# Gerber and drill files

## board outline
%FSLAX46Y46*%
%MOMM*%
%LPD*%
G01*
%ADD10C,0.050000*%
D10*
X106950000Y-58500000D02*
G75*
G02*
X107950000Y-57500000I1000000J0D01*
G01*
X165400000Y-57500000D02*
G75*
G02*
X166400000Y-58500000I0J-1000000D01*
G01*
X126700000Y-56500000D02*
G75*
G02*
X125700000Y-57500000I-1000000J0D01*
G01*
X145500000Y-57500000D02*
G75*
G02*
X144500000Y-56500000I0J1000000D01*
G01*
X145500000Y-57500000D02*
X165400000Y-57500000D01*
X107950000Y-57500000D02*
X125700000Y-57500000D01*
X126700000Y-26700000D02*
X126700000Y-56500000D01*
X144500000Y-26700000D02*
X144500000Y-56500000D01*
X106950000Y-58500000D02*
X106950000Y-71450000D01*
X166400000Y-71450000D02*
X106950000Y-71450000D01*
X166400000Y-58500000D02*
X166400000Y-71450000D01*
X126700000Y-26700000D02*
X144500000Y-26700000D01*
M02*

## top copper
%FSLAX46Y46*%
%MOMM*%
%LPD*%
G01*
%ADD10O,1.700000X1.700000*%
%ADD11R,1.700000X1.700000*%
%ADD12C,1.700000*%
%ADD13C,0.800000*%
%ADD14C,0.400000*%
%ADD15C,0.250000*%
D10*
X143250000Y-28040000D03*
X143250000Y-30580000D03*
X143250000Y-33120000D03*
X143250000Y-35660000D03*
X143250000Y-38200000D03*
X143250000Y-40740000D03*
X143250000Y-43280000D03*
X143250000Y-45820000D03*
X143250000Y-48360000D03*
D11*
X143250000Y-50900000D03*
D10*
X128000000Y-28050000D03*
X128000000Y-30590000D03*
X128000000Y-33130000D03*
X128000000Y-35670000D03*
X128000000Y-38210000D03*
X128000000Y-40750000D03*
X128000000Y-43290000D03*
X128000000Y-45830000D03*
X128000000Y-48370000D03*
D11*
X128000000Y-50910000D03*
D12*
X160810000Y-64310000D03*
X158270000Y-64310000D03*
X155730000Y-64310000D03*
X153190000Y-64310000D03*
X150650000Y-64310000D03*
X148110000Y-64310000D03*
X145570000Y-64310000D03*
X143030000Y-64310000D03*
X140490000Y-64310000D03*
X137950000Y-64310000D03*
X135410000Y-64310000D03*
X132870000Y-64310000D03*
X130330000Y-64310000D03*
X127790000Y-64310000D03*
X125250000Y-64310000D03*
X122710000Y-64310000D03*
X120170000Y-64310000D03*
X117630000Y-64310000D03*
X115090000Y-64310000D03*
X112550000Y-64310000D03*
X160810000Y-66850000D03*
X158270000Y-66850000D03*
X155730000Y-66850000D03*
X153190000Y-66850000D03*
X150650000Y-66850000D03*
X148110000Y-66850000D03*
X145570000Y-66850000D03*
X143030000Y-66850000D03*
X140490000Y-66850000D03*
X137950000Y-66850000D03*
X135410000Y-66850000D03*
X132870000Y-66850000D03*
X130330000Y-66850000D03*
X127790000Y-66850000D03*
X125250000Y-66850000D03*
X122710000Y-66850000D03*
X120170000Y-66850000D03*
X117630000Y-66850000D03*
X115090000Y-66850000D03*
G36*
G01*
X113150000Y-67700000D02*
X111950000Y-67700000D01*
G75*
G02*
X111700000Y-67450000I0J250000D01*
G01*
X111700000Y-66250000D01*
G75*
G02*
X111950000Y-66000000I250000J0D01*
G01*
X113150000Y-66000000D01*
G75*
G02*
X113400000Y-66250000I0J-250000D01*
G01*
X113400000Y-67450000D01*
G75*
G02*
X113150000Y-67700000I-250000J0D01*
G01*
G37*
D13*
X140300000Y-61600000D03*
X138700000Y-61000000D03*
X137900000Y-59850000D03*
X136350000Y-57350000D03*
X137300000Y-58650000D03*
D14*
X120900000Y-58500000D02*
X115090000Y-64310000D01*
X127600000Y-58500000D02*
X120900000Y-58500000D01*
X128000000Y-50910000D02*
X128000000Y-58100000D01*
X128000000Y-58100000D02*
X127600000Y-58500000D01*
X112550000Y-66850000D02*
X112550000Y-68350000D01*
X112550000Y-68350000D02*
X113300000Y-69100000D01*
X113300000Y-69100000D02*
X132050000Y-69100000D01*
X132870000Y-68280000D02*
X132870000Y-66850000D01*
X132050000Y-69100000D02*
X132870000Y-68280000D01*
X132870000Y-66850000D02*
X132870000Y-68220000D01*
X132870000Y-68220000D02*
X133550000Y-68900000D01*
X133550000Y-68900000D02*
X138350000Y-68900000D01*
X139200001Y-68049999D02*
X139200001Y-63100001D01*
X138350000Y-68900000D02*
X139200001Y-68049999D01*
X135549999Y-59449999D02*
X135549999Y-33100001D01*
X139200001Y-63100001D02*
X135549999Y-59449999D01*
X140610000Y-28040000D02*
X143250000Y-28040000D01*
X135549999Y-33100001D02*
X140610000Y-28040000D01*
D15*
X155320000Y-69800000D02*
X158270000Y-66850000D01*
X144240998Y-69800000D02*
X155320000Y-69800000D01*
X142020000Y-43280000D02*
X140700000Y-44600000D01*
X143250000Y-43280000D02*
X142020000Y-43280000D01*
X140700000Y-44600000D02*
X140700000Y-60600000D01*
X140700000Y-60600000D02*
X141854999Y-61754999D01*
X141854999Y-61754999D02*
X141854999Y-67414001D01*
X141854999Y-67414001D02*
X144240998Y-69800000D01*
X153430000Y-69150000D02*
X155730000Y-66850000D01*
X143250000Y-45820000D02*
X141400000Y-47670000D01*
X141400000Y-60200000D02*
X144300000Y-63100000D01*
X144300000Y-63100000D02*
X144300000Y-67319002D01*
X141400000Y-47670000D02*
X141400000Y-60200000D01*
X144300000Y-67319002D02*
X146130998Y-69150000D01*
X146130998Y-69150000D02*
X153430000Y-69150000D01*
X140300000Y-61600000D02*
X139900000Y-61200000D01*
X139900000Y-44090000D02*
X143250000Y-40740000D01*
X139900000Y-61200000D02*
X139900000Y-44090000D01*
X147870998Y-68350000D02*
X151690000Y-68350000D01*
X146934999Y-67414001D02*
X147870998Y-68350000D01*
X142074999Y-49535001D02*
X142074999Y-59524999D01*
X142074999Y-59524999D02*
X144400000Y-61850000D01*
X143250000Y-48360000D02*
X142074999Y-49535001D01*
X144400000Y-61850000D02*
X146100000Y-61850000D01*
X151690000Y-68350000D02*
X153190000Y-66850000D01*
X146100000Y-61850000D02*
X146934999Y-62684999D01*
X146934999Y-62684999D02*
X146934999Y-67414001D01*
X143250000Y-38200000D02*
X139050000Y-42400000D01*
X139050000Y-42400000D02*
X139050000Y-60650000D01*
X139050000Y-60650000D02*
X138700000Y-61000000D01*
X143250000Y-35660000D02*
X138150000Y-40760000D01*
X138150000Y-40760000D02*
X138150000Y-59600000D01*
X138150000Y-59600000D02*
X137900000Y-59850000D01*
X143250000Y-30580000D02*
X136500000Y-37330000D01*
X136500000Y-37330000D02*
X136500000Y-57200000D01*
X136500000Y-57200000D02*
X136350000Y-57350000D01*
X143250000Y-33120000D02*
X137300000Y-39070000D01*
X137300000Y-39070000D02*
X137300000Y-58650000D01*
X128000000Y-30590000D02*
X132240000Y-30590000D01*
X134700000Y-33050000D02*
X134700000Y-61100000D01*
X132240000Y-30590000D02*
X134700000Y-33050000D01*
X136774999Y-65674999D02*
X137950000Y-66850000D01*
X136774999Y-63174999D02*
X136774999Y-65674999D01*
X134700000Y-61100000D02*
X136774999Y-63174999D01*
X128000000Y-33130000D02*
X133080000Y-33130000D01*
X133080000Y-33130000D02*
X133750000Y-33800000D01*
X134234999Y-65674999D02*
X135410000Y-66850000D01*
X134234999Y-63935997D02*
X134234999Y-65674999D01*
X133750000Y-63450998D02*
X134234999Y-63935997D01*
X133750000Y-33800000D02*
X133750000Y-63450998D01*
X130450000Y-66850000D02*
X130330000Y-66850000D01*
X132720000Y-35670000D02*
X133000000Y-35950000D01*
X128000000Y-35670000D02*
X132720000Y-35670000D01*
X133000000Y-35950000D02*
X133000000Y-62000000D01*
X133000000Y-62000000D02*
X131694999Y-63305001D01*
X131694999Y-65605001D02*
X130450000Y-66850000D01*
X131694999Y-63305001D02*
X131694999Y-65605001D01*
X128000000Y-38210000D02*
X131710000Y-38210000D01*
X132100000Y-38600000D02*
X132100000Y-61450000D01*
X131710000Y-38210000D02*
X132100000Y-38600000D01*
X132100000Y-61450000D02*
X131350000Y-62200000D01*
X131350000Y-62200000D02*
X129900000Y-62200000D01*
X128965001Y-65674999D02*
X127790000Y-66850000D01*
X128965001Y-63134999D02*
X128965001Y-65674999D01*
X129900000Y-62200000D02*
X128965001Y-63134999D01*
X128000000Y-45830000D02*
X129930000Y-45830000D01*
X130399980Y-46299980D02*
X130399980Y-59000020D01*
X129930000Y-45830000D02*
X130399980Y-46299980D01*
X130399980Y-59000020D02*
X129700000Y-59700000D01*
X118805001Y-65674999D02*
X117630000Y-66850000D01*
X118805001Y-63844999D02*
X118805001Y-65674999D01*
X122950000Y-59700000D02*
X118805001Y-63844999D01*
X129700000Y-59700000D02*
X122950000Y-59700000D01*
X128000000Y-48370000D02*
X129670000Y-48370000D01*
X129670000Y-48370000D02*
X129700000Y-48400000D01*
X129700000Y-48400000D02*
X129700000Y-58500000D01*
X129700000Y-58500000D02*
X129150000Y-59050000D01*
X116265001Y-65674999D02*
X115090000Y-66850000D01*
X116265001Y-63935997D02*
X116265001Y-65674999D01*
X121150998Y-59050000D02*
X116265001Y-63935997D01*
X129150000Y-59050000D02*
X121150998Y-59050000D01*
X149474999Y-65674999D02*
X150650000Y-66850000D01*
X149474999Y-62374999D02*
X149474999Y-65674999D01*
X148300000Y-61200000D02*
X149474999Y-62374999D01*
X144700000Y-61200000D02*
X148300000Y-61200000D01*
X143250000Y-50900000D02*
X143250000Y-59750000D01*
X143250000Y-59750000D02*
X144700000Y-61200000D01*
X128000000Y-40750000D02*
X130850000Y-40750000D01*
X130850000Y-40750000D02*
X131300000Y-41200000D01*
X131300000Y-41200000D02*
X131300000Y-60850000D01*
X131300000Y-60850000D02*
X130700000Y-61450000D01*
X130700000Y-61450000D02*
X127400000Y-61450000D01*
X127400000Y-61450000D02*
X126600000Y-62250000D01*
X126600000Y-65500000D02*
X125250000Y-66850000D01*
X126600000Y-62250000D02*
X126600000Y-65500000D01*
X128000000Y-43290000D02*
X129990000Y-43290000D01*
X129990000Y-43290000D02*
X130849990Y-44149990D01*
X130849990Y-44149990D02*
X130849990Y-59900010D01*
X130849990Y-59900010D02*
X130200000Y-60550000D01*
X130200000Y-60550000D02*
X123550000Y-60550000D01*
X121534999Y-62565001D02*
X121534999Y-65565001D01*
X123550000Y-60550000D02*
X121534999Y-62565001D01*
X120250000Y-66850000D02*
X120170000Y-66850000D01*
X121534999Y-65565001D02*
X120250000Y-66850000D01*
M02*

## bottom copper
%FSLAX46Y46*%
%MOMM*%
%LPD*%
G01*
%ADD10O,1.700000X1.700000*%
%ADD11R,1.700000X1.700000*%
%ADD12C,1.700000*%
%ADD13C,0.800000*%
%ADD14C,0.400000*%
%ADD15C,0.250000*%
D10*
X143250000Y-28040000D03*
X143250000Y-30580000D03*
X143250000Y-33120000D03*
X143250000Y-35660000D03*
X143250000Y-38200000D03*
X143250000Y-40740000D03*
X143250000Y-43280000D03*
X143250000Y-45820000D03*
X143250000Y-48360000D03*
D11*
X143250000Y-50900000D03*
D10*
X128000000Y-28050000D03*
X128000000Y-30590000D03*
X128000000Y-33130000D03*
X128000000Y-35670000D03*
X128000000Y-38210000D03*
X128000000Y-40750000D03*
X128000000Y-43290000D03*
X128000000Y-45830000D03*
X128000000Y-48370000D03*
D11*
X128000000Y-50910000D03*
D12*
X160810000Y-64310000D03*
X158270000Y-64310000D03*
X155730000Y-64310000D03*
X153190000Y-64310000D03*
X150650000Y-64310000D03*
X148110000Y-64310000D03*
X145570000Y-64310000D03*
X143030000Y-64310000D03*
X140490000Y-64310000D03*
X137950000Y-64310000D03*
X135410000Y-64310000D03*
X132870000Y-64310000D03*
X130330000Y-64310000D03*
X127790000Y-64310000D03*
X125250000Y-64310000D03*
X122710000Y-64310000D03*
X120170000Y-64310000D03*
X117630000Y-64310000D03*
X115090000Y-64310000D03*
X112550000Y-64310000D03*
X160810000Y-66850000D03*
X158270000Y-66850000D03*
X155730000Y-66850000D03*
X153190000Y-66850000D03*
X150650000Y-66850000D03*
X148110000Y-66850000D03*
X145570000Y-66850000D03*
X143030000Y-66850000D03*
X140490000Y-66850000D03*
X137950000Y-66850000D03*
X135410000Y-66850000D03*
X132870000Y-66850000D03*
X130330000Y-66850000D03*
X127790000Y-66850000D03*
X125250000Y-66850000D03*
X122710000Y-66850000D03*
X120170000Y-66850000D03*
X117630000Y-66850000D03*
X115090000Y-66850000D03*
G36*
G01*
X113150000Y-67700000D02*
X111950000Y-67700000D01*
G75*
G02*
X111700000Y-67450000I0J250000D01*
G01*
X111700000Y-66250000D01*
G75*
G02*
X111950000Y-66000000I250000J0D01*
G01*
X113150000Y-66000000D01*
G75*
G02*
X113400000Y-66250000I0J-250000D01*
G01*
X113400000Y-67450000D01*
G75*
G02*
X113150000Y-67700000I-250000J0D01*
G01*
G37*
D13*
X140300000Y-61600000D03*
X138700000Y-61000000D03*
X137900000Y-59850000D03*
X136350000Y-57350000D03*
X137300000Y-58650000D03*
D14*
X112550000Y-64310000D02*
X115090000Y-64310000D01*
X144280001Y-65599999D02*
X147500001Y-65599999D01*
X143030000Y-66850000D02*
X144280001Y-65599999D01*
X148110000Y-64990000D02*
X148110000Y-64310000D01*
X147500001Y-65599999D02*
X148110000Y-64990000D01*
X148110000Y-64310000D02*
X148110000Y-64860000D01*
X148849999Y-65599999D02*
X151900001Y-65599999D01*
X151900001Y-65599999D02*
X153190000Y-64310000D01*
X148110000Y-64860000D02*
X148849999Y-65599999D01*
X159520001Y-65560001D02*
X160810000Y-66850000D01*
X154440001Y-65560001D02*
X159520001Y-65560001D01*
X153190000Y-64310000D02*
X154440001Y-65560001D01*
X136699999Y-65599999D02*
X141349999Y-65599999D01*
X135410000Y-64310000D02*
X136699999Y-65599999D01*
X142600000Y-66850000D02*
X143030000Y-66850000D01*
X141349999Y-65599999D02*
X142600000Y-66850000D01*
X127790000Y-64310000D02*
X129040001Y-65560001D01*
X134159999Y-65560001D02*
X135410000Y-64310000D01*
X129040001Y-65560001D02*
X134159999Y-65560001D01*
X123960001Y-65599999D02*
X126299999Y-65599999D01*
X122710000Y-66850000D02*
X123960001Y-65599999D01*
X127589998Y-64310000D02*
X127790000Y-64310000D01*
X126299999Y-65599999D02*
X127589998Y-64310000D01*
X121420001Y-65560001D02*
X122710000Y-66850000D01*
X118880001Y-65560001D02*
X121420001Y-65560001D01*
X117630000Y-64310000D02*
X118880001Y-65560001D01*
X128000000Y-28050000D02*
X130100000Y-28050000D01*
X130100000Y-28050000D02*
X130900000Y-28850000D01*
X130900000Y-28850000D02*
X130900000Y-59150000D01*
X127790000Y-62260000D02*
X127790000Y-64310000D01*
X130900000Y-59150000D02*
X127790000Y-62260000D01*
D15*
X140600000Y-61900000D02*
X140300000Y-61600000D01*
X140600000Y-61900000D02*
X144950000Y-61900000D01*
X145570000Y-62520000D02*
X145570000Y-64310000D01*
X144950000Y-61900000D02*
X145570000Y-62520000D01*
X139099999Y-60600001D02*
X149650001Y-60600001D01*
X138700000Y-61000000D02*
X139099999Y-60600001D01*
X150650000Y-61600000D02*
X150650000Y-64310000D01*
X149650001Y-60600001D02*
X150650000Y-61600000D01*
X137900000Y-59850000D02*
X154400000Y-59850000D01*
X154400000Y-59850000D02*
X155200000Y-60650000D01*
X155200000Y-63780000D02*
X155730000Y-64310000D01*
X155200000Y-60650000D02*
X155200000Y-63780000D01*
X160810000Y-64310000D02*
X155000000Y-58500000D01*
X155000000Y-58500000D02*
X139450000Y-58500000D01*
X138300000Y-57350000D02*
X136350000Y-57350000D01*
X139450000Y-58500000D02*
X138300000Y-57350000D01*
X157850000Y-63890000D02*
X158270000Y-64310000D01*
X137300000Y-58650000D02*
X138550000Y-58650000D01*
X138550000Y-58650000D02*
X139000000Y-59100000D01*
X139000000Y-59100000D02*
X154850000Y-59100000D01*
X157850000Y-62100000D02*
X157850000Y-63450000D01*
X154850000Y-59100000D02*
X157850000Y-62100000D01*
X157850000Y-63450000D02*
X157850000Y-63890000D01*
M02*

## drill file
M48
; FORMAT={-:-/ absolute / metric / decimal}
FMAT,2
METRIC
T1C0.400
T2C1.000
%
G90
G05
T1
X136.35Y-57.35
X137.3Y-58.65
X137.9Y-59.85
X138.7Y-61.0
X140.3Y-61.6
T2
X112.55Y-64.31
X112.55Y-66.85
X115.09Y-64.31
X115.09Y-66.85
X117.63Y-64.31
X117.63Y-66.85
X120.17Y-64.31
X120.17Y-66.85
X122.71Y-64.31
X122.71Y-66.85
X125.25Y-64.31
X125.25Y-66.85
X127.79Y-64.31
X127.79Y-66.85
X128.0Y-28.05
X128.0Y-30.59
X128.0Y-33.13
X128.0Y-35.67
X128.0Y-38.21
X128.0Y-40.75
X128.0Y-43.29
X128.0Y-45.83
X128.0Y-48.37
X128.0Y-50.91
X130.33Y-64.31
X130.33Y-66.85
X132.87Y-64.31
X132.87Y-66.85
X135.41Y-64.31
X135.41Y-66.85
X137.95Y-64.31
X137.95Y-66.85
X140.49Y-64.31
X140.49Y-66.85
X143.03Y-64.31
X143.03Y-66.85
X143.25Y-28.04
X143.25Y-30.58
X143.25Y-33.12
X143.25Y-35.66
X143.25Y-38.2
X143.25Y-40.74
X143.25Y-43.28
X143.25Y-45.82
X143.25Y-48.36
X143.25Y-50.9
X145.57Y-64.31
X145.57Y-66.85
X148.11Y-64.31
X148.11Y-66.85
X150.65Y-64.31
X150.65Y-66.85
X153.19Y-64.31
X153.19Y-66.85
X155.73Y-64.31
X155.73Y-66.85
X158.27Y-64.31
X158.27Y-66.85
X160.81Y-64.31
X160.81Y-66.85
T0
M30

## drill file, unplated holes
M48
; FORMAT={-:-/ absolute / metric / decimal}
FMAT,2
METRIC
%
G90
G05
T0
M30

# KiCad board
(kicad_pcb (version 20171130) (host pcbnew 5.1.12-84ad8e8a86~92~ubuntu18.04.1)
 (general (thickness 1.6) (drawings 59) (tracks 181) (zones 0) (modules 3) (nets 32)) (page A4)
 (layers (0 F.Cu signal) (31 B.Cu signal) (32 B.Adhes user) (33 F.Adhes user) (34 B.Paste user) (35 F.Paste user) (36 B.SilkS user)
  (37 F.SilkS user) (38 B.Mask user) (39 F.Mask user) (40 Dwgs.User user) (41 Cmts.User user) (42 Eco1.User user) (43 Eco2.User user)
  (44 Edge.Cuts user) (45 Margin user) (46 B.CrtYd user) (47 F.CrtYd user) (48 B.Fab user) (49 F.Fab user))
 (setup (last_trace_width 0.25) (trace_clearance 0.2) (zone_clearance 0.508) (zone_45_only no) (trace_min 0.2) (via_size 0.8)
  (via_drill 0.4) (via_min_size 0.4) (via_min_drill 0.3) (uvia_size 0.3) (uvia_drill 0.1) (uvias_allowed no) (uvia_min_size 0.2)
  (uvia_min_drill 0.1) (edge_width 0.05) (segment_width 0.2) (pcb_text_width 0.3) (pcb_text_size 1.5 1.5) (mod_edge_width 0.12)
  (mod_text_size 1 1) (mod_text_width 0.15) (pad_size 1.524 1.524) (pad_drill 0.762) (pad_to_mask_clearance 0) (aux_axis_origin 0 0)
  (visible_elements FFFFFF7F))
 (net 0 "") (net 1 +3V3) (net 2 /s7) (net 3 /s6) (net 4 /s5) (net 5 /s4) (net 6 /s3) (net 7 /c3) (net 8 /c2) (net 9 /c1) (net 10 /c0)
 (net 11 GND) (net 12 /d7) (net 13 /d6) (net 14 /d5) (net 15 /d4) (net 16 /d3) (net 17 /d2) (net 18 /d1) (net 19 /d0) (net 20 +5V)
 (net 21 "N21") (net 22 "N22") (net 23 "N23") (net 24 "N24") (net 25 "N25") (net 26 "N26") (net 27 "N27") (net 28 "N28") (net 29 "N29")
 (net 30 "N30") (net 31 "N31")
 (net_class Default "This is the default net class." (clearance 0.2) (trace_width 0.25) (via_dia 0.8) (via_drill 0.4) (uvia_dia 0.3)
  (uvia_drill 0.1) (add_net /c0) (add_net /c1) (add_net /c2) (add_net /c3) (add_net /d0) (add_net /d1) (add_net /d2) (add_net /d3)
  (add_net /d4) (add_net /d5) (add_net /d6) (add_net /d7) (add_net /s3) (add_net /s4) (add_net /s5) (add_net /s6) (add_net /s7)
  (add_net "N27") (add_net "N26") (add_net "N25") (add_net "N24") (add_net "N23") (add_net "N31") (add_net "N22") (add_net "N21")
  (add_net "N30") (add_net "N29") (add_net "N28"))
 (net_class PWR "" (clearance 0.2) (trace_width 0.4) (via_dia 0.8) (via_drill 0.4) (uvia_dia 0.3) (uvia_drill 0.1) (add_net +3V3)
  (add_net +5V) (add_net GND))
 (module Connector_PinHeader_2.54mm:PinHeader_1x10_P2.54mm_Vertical (layer F.Cu) (at 143.25 50.9 180)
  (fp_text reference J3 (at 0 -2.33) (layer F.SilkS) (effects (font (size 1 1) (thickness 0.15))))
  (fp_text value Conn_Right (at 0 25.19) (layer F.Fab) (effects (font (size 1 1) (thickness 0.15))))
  (pad 10 thru_hole oval (at 0 22.86 180) (size 1.7 1.7) (drill 1) (layers *.Cu *.Mask) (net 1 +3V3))
  (pad 9 thru_hole oval (at 0 20.32 180) (size 1.7 1.7) (drill 1) (layers *.Cu *.Mask) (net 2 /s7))
  (pad 8 thru_hole oval (at 0 17.78 180) (size 1.7 1.7) (drill 1) (layers *.Cu *.Mask) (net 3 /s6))
  (pad 7 thru_hole oval (at 0 15.24 180) (size 1.7 1.7) (drill 1) (layers *.Cu *.Mask) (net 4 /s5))
  (pad 6 thru_hole oval (at 0 12.7 180) (size 1.7 1.7) (drill 1) (layers *.Cu *.Mask) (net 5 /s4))
  (pad 5 thru_hole oval (at 0 10.16 180) (size 1.7 1.7) (drill 1) (layers *.Cu *.Mask) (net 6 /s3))
  (pad 4 thru_hole oval (at 0 7.62 180) (size 1.7 1.7) (drill 1) (layers *.Cu *.Mask) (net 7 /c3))
  (pad 3 thru_hole oval (at 0 5.08 180) (size 1.7 1.7) (drill 1) (layers *.Cu *.Mask) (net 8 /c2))
  (pad 2 thru_hole oval (at 0 2.54 180) (size 1.7 1.7) (drill 1) (layers *.Cu *.Mask) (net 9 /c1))
  (pad 1 thru_hole rect (at 0 0 180) (size 1.7 1.7) (drill 1) (layers *.Cu *.Mask) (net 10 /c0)))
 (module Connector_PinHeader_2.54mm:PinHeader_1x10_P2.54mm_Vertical (layer F.Cu) (at 128 50.91 180)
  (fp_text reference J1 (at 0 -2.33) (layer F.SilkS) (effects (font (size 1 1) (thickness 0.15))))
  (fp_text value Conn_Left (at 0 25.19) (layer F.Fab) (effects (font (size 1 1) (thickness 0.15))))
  (pad 10 thru_hole oval (at 0 22.86 180) (size 1.7 1.7) (drill 1) (layers *.Cu *.Mask) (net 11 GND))
  (pad 9 thru_hole oval (at 0 20.32 180) (size 1.7 1.7) (drill 1) (layers *.Cu *.Mask) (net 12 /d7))
  (pad 8 thru_hole oval (at 0 17.78 180) (size 1.7 1.7) (drill 1) (layers *.Cu *.Mask) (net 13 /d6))
  (pad 7 thru_hole oval (at 0 15.24 180) (size 1.7 1.7) (drill 1) (layers *.Cu *.Mask) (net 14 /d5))
  (pad 6 thru_hole oval (at 0 12.7 180) (size 1.7 1.7) (drill 1) (layers *.Cu *.Mask) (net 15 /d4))
  (pad 5 thru_hole oval (at 0 10.16 180) (size 1.7 1.7) (drill 1) (layers *.Cu *.Mask) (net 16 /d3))
  (pad 4 thru_hole oval (at 0 7.62 180) (size 1.7 1.7) (drill 1) (layers *.Cu *.Mask) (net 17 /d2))
  (pad 3 thru_hole oval (at 0 5.08 180) (size 1.7 1.7) (drill 1) (layers *.Cu *.Mask) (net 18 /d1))
  (pad 2 thru_hole oval (at 0 2.54 180) (size 1.7 1.7) (drill 1) (layers *.Cu *.Mask) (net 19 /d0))
  (pad 1 thru_hole rect (at 0 0 180) (size 1.7 1.7) (drill 1) (layers *.Cu *.Mask) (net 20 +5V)))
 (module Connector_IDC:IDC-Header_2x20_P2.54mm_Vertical (layer F.Cu) (at 112.55 66.85 90)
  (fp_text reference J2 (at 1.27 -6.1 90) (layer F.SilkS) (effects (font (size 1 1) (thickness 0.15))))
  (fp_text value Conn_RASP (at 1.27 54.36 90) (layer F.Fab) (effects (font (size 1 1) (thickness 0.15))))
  (pad 40 thru_hole circle (at 2.54 48.26 90) (size 1.7 1.7) (drill 1) (layers *.Cu *.Mask) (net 2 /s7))
  (pad 38 thru_hole circle (at 2.54 45.72 90) (size 1.7 1.7) (drill 1) (layers *.Cu *.Mask) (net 3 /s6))
  (pad 36 thru_hole circle (at 2.54 43.18 90) (size 1.7 1.7) (drill 1) (layers *.Cu *.Mask) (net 4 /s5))
  (pad 34 thru_hole circle (at 2.54 40.64 90) (size 1.7 1.7) (drill 1) (layers *.Cu *.Mask) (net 11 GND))
  (pad 32 thru_hole circle (at 2.54 38.1 90) (size 1.7 1.7) (drill 1) (layers *.Cu *.Mask) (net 5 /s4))
  (pad 30 thru_hole circle (at 2.54 35.56 90) (size 1.7 1.7) (drill 1) (layers *.Cu *.Mask) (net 11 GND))
  (pad 28 thru_hole circle (at 2.54 33.02 90) (size 1.7 1.7) (drill 1) (layers *.Cu *.Mask) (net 6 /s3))
  (pad 26 thru_hole circle (at 2.54 30.48 90) (size 1.7 1.7) (drill 1) (layers *.Cu *.Mask) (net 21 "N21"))
  (pad 24 thru_hole circle (at 2.54 27.94 90) (size 1.7 1.7) (drill 1) (layers *.Cu *.Mask) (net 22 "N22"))
  (pad 22 thru_hole circle (at 2.54 25.4 90) (size 1.7 1.7) (drill 1) (layers *.Cu *.Mask) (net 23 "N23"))
  (pad 20 thru_hole circle (at 2.54 22.86 90) (size 1.7 1.7) (drill 1) (layers *.Cu *.Mask) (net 11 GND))
  (pad 18 thru_hole circle (at 2.54 20.32 90) (size 1.7 1.7) (drill 1) (layers *.Cu *.Mask) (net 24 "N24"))
  (pad 16 thru_hole circle (at 2.54 17.78 90) (size 1.7 1.7) (drill 1) (layers *.Cu *.Mask) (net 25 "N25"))
  (pad 14 thru_hole circle (at 2.54 15.24 90) (size 1.7 1.7) (drill 1) (layers *.Cu *.Mask) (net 11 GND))
  (pad 12 thru_hole circle (at 2.54 12.7 90) (size 1.7 1.7) (drill 1) (layers *.Cu *.Mask) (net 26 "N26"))
  (pad 10 thru_hole circle (at 2.54 10.16 90) (size 1.7 1.7) (drill 1) (layers *.Cu *.Mask) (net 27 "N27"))
  (pad 8 thru_hole circle (at 2.54 7.62 90) (size 1.7 1.7) (drill 1) (layers *.Cu *.Mask) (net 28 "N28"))
  (pad 6 thru_hole circle (at 2.54 5.08 90) (size 1.7 1.7) (drill 1) (layers *.Cu *.Mask) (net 11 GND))
  (pad 4 thru_hole circle (at 2.54 2.54 90) (size 1.7 1.7) (drill 1) (layers *.Cu *.Mask) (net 20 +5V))
  (pad 2 thru_hole circle (at 2.54 0 90) (size 1.7 1.7) (drill 1) (layers *.Cu *.Mask) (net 20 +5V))
  (pad 39 thru_hole circle (at 0 48.26 90) (size 1.7 1.7) (drill 1) (layers *.Cu *.Mask) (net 11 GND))
  (pad 37 thru_hole circle (at 0 45.72 90) (size 1.7 1.7) (drill 1) (layers *.Cu *.Mask) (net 7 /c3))
  (pad 35 thru_hole circle (at 0 43.18 90) (size 1.7 1.7) (drill 1) (layers *.Cu *.Mask) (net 8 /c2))
  (pad 33 thru_hole circle (at 0 40.64 90) (size 1.7 1.7) (drill 1) (layers *.Cu *.Mask) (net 9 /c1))
  (pad 31 thru_hole circle (at 0 38.1 90) (size 1.7 1.7) (drill 1) (layers *.Cu *.Mask) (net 10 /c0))
  (pad 29 thru_hole circle (at 0 35.56 90) (size 1.7 1.7) (drill 1) (layers *.Cu *.Mask) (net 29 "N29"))
  (pad 27 thru_hole circle (at 0 33.02 90) (size 1.7 1.7) (drill 1) (layers *.Cu *.Mask) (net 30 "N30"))
  (pad 25 thru_hole circle (at 0 30.48 90) (size 1.7 1.7) (drill 1) (layers *.Cu *.Mask) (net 11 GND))
  (pad 23 thru_hole circle (at 0 27.94 90) (size 1.7 1.7) (drill 1) (layers *.Cu *.Mask) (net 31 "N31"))
  (pad 21 thru_hole circle (at 0 25.4 90) (size 1.7 1.7) (drill 1) (layers *.Cu *.Mask) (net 12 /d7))
  (pad 19 thru_hole circle (at 0 22.86 90) (size 1.7 1.7) (drill 1) (layers *.Cu *.Mask) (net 13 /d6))
  (pad 17 thru_hole circle (at 0 20.32 90) (size 1.7 1.7) (drill 1) (layers *.Cu *.Mask) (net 1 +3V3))
  (pad 15 thru_hole circle (at 0 17.78 90) (size 1.7 1.7) (drill 1) (layers *.Cu *.Mask) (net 14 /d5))
  (pad 13 thru_hole circle (at 0 15.24 90) (size 1.7 1.7) (drill 1) (layers *.Cu *.Mask) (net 15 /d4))
  (pad 11 thru_hole circle (at 0 12.7 90) (size 1.7 1.7) (drill 1) (layers *.Cu *.Mask) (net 16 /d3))
  (pad 9 thru_hole circle (at 0 10.16 90) (size 1.7 1.7) (drill 1) (layers *.Cu *.Mask) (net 11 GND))
  (pad 7 thru_hole circle (at 0 7.62 90) (size 1.7 1.7) (drill 1) (layers *.Cu *.Mask) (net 17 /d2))
  (pad 5 thru_hole circle (at 0 5.08 90) (size 1.7 1.7) (drill 1) (layers *.Cu *.Mask) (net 18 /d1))
  (pad 3 thru_hole circle (at 0 2.54 90) (size 1.7 1.7) (drill 1) (layers *.Cu *.Mask) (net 19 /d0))
  (pad 1 thru_hole roundrect (at 0 0 90) (size 1.7 1.7) (drill 1) (layers *.Cu *.Mask) (roundrect_rratio 0.1470588235294118) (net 1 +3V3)))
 (gr_arc (start 107.95 58.5) (end 107.95 57.5) (angle -90) (layer Edge.Cuts) (width 0.05))
 (gr_arc (start 165.4 58.5) (end 166.4 58.5) (angle -90) (layer Edge.Cuts) (width 0.05))
 (gr_arc (start 125.7 56.5) (end 125.7 57.5) (angle -90) (layer Edge.Cuts) (width 0.05))
 (gr_arc (start 145.5 56.5) (end 144.5 56.5) (angle -90) (layer Edge.Cuts) (width 0.05))
 (gr_line (start 145.5 57.5) (end 165.4 57.5) (layer Edge.Cuts) (width 0.05))
 (gr_line (start 107.95 57.5) (end 125.7 57.5) (layer Edge.Cuts) (width 0.05))
 (gr_line (start 126.7 26.7) (end 126.7 56.5) (layer Edge.Cuts) (width 0.05))
 (gr_line (start 144.5 26.7) (end 144.5 56.5) (layer Edge.Cuts) (width 0.05))
 (gr_line (start 106.95 58.5) (end 106.95 71.45) (layer Edge.Cuts) (width 0.05))
 (gr_line (start 166.4 71.45) (end 106.95 71.45) (layer Edge.Cuts) (width 0.05))
 (gr_line (start 166.4 58.5) (end 166.4 71.45) (layer Edge.Cuts) (width 0.05))
 (gr_line (start 126.7 26.7) (end 144.5 26.7) (layer Edge.Cuts) (width 0.05))
 (segment (start 112.55 64.31) (end 115.09 64.31) (width 0.4) (layer B.Cu) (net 20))
 (segment (start 120.9 58.5) (end 115.09 64.31) (width 0.4) (layer F.Cu) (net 20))
 (segment (start 127.6 58.5) (end 120.9 58.5) (width 0.4) (layer F.Cu) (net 20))
 (segment (start 128 50.91) (end 128 58.1) (width 0.4) (layer F.Cu) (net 20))
 (segment (start 128 58.1) (end 127.6 58.5) (width 0.4) (layer F.Cu) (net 20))
 (segment (start 144.280001 65.599999) (end 147.500001 65.599999) (width 0.4) (layer B.Cu) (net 11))
 (segment (start 143.03 66.85) (end 144.280001 65.599999) (width 0.4) (layer B.Cu) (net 11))
 (segment (start 148.11 64.99) (end 148.11 64.31) (width 0.4) (layer B.Cu) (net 11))
 (segment (start 147.500001 65.599999) (end 148.11 64.99) (width 0.4) (layer B.Cu) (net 11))
 (segment (start 148.11 64.31) (end 148.11 64.86) (width 0.4) (layer B.Cu) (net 11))
 (segment (start 148.849999 65.599999) (end 151.900001 65.599999) (width 0.4) (layer B.Cu) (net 11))
 (segment (start 151.900001 65.599999) (end 153.19 64.31) (width 0.4) (layer B.Cu) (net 11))
 (segment (start 148.11 64.86) (end 148.849999 65.599999) (width 0.4) (layer B.Cu) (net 11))
 (segment (start 159.520001 65.560001) (end 160.81 66.85) (width 0.4) (layer B.Cu) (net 11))
 (segment (start 154.440001 65.560001) (end 159.520001 65.560001) (width 0.4) (layer B.Cu) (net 11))
 (segment (start 153.19 64.31) (end 154.440001 65.560001) (width 0.4) (layer B.Cu) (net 11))
 (segment (start 136.699999 65.599999) (end 141.349999 65.599999) (width 0.4) (layer B.Cu) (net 11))
 (segment (start 135.41 64.31) (end 136.699999 65.599999) (width 0.4) (layer B.Cu) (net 11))
 (segment (start 142.6 66.85) (end 143.03 66.85) (width 0.4) (layer B.Cu) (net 11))
 (segment (start 141.349999 65.599999) (end 142.6 66.85) (width 0.4) (layer B.Cu) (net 11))
 (segment (start 127.79 64.31) (end 129.040001 65.560001) (width 0.4) (layer B.Cu) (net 11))
 (segment (start 134.159999 65.560001) (end 135.41 64.31) (width 0.4) (layer B.Cu) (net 11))
 (segment (start 129.040001 65.560001) (end 134.159999 65.560001) (width 0.4) (layer B.Cu) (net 11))
 (segment (start 123.960001 65.599999) (end 126.299999 65.599999) (width 0.4) (layer B.Cu) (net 11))
 (segment (start 122.71 66.85) (end 123.960001 65.599999) (width 0.4) (layer B.Cu) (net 11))
 (segment (start 127.589998 64.31) (end 127.79 64.31) (width 0.4) (layer B.Cu) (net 11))
 (segment (start 126.299999 65.599999) (end 127.589998 64.31) (width 0.4) (layer B.Cu) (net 11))
 (segment (start 121.420001 65.560001) (end 122.71 66.85) (width 0.4) (layer B.Cu) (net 11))
 (segment (start 118.880001 65.560001) (end 121.420001 65.560001) (width 0.4) (layer B.Cu) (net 11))
 (segment (start 117.63 64.31) (end 118.880001 65.560001) (width 0.4) (layer B.Cu) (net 11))
 (segment (start 128 28.05) (end 130.1 28.05) (width 0.4) (layer B.Cu) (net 11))
 (segment (start 130.1 28.05) (end 130.9 28.85) (width 0.4) (layer B.Cu) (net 11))
 (segment (start 130.9 28.85) (end 130.9 59.15) (width 0.4) (layer B.Cu) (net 11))
 (segment (start 127.79 62.26) (end 127.79 64.31) (width 0.4) (layer B.Cu) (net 11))
 (segment (start 130.9 59.15) (end 127.79 62.26) (width 0.4) (layer B.Cu) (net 11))
 (segment (start 112.55 66.85) (end 112.55 68.35) (width 0.4) (layer F.Cu) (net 1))
 (segment (start 112.55 68.35) (end 113.3 69.1) (width 0.4) (layer F.Cu) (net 1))
 (segment (start 113.3 69.1) (end 132.05 69.1) (width 0.4) (layer F.Cu) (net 1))
 (segment (start 132.87 68.28) (end 132.87 66.85) (width 0.4) (layer F.Cu) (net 1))
 (segment (start 132.05 69.1) (end 132.87 68.28) (width 0.4) (layer F.Cu) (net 1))
 (segment (start 132.87 66.85) (end 132.87 68.22) (width 0.4) (layer F.Cu) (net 1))
 (segment (start 132.87 68.22) (end 133.55 68.9) (width 0.4) (layer F.Cu) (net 1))
 (segment (start 133.55 68.9) (end 138.35 68.9) (width 0.4) (layer F.Cu) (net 1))
 (segment (start 139.200001 68.049999) (end 139.200001 63.100001) (width 0.4) (layer F.Cu) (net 1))
 (segment (start 138.35 68.9) (end 139.200001 68.049999) (width 0.4) (layer F.Cu) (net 1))
 (segment (start 135.549999 59.449999) (end 135.549999 33.100001) (width 0.4) (layer F.Cu) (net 1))
 (segment (start 139.200001 63.100001) (end 135.549999 59.449999) (width 0.4) (layer F.Cu) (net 1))
 (segment (start 140.61 28.04) (end 143.25 28.04) (width 0.4) (layer F.Cu) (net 1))
 (segment (start 135.549999 33.100001) (end 140.61 28.04) (width 0.4) (layer F.Cu) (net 1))
 (segment (start 155.32 69.8) (end 158.27 66.85) (width 0.25) (layer F.Cu) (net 7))
 (segment (start 144.240998 69.8) (end 155.32 69.8) (width 0.25) (layer F.Cu) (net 7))
 (segment (start 142.02 43.28) (end 140.7 44.6) (width 0.25) (layer F.Cu) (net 7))
 (segment (start 143.25 43.28) (end 142.02 43.28) (width 0.25) (layer F.Cu) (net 7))
 (segment (start 140.7 44.6) (end 140.7 60.6) (width 0.25) (layer F.Cu) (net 7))
 (segment (start 140.7 60.6) (end 141.854999 61.754999) (width 0.25) (layer F.Cu) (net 7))
 (segment (start 141.854999 61.754999) (end 141.854999 67.414001) (width 0.25) (layer F.Cu) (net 7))
 (segment (start 141.854999 67.414001) (end 144.240998 69.8) (width 0.25) (layer F.Cu) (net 7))
 (segment (start 153.43 69.15) (end 155.73 66.85) (width 0.25) (layer F.Cu) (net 8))
 (segment (start 143.25 45.82) (end 141.4 47.67) (width 0.25) (layer F.Cu) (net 8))
 (segment (start 141.4 60.2) (end 144.3 63.1) (width 0.25) (layer F.Cu) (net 8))
 (segment (start 144.3 63.1) (end 144.3 67.319002) (width 0.25) (layer F.Cu) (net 8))
 (segment (start 141.4 47.67) (end 141.4 60.2) (width 0.25) (layer F.Cu) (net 8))
 (segment (start 144.3 67.319002) (end 146.130998 69.15) (width 0.25) (layer F.Cu) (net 8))
 (segment (start 146.130998 69.15) (end 153.43 69.15) (width 0.25) (layer F.Cu) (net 8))
 (via (at 140.3 61.6) (size 0.8) (drill 0.4) (layers F.Cu B.Cu) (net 6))
 (segment (start 140.6 61.9) (end 140.3 61.6) (width 0.25) (layer B.Cu) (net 6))
 (segment (start 140.3 61.6) (end 139.9 61.2) (width 0.25) (layer F.Cu) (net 6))
 (segment (start 139.9 44.09) (end 143.25 40.74) (width 0.25) (layer F.Cu) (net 6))
 (segment (start 139.9 61.2) (end 139.9 44.09) (width 0.25) (layer F.Cu) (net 6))
 (segment (start 140.6 61.9) (end 144.95 61.9) (width 0.25) (layer B.Cu) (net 6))
 (segment (start 145.57 62.52) (end 145.57 64.31) (width 0.25) (layer B.Cu) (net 6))
 (segment (start 144.95 61.9) (end 145.57 62.52) (width 0.25) (layer B.Cu) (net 6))
 (segment (start 147.870998 68.35) (end 151.69 68.35) (width 0.25) (layer F.Cu) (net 9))
 (segment (start 146.934999 67.414001) (end 147.870998 68.35) (width 0.25) (layer F.Cu) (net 9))
 (segment (start 142.074999 49.535001) (end 142.074999 59.524999) (width 0.25) (layer F.Cu) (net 9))
 (segment (start 142.074999 59.524999) (end 144.4 61.85) (width 0.25) (layer F.Cu) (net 9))
 (segment (start 143.25 48.36) (end 142.074999 49.535001) (width 0.25) (layer F.Cu) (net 9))
 (segment (start 144.4 61.85) (end 146.1 61.85) (width 0.25) (layer F.Cu) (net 9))
 (segment (start 151.69 68.35) (end 153.19 66.85) (width 0.25) (layer F.Cu) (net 9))
 (segment (start 146.1 61.85) (end 146.934999 62.684999) (width 0.25) (layer F.Cu) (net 9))
 (segment (start 146.934999 62.684999) (end 146.934999 67.414001) (width 0.25) (layer F.Cu) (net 9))
 (segment (start 143.25 38.2) (end 139.05 42.4) (width 0.25) (layer F.Cu) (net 5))
 (via (at 138.7 61) (size 0.8) (drill 0.4) (layers F.Cu B.Cu) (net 5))
 (segment (start 139.05 42.4) (end 139.05 60.65) (width 0.25) (layer F.Cu) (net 5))
 (segment (start 139.05 60.65) (end 138.7 61) (width 0.25) (layer F.Cu) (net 5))
 (segment (start 139.099999 60.600001) (end 149.650001 60.600001) (width 0.25) (layer B.Cu) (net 5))
 (segment (start 138.7 61) (end 139.099999 60.600001) (width 0.25) (layer B.Cu) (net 5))
 (segment (start 150.65 61.6) (end 150.65 64.31) (width 0.25) (layer B.Cu) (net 5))
 (segment (start 149.650001 60.600001) (end 150.65 61.6) (width 0.25) (layer B.Cu) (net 5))
 (segment (start 143.25 35.66) (end 138.15 40.76) (width 0.25) (layer F.Cu) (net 4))
 (segment (start 138.15 40.76) (end 138.15 59.6) (width 0.25) (layer F.Cu) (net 4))
 (via (at 137.9 59.85) (size 0.8) (drill 0.4) (layers F.Cu B.Cu) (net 4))
 (segment (start 138.15 59.6) (end 137.9 59.85) (width 0.25) (layer F.Cu) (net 4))
 (segment (start 137.9 59.85) (end 154.4 59.85) (width 0.25) (layer B.Cu) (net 4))
 (segment (start 154.4 59.85) (end 155.2 60.65) (width 0.25) (layer B.Cu) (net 4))
 (segment (start 155.2 63.78) (end 155.73 64.31) (width 0.25) (layer B.Cu) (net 4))
 (segment (start 155.2 60.65) (end 155.2 63.78) (width 0.25) (layer B.Cu) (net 4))
 (segment (start 143.25 30.58) (end 136.5 37.33) (width 0.25) (layer F.Cu) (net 2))
 (via (at 136.35 57.35) (size 0.8) (drill 0.4) (layers F.Cu B.Cu) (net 2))
 (segment (start 136.5 37.33) (end 136.5 57.2) (width 0.25) (layer F.Cu) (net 2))
 (segment (start 136.5 57.2) (end 136.35 57.35) (width 0.25) (layer F.Cu) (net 2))
 (segment (start 160.81 64.31) (end 155 58.5) (width 0.25) (layer B.Cu) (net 2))
 (segment (start 155 58.5) (end 139.45 58.5) (width 0.25) (layer B.Cu) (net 2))
 (segment (start 138.3 57.35) (end 136.35 57.35) (width 0.25) (layer B.Cu) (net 2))
 (segment (start 139.45 58.5) (end 138.3 57.35) (width 0.25) (layer B.Cu) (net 2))
 (segment (start 143.25 33.12) (end 137.3 39.07) (width 0.25) (layer F.Cu) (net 3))
 (via (at 137.3 58.65) (size 0.8) (drill 0.4) (layers F.Cu B.Cu) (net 3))
 (segment (start 137.3 39.07) (end 137.3 58.65) (width 0.25) (layer F.Cu) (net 3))
 (segment (start 157.85 63.89) (end 158.27 64.31) (width 0.25) (layer B.Cu) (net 3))
 (segment (start 137.3 58.65) (end 138.55 58.65) (width 0.25) (layer B.Cu) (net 3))
 (segment (start 138.55 58.65) (end 139 59.1) (width 0.25) (layer B.Cu) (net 3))
 (segment (start 139 59.1) (end 154.85 59.1) (width 0.25) (layer B.Cu) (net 3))
 (segment (start 157.85 62.1) (end 157.85 63.45) (width 0.25) (layer B.Cu) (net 3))
 (segment (start 154.85 59.1) (end 157.85 62.1) (width 0.25) (layer B.Cu) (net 3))
 (segment (start 157.85 63.45) (end 157.85 63.89) (width 0.25) (layer B.Cu) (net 3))
 (segment (start 128 30.59) (end 132.24 30.59) (width 0.25) (layer F.Cu) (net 12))
 (segment (start 134.7 33.05) (end 134.7 61.1) (width 0.25) (layer F.Cu) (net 12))
 (segment (start 132.24 30.59) (end 134.7 33.05) (width 0.25) (layer F.Cu) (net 12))
 (segment (start 136.774999 65.674999) (end 137.95 66.85) (width 0.25) (layer F.Cu) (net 12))
 (segment (start 136.774999 63.174999) (end 136.774999 65.674999) (width 0.25) (layer F.Cu) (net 12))
 (segment (start 134.7 61.1) (end 136.774999 63.174999) (width 0.25) (layer F.Cu) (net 12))
 (segment (start 128 33.13) (end 133.08 33.13) (width 0.25) (layer F.Cu) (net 13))
 (segment (start 133.08 33.13) (end 133.75 33.8) (width 0.25) (layer F.Cu) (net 13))
 (segment (start 134.234999 65.674999) (end 135.41 66.85) (width 0.25) (layer F.Cu) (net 13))
 (segment (start 134.234999 63.935997) (end 134.234999 65.674999) (width 0.25) (layer F.Cu) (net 13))
 (segment (start 133.75 63.450998) (end 134.234999 63.935997) (width 0.25) (layer F.Cu) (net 13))
 (segment (start 133.75 33.8) (end 133.75 63.450998) (width 0.25) (layer F.Cu) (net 13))
 (segment (start 130.45 66.85) (end 130.33 66.85) (width 0.25) (layer F.Cu) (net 14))
 (segment (start 132.72 35.67) (end 133 35.95) (width 0.25) (layer F.Cu) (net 14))
 (segment (start 128 35.67) (end 132.72 35.67) (width 0.25) (layer F.Cu) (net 14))
 (segment (start 133 35.95) (end 133 62) (width 0.25) (layer F.Cu) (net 14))
 (segment (start 133 62) (end 131.694999 63.305001) (width 0.25) (layer F.Cu) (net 14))
 (segment (start 131.694999 65.605001) (end 130.45 66.85) (width 0.25) (layer F.Cu) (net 14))
 (segment (start 131.694999 63.305001) (end 131.694999 65.605001) (width 0.25) (layer F.Cu) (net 14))
 (segment (start 128 38.21) (end 131.71 38.21) (width 0.25) (layer F.Cu) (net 15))
 (segment (start 132.1 38.6) (end 132.1 61.45) (width 0.25) (layer F.Cu) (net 15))
 (segment (start 131.71 38.21) (end 132.1 38.6) (width 0.25) (layer F.Cu) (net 15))
 (segment (start 132.1 61.45) (end 131.35 62.2) (width 0.25) (layer F.Cu) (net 15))
 (segment (start 131.35 62.2) (end 129.9 62.2) (width 0.25) (layer F.Cu) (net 15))
 (segment (start 128.965001 65.674999) (end 127.79 66.85) (width 0.25) (layer F.Cu) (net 15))
 (segment (start 128.965001 63.134999) (end 128.965001 65.674999) (width 0.25) (layer F.Cu) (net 15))
 (segment (start 129.9 62.2) (end 128.965001 63.134999) (width 0.25) (layer F.Cu) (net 15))
 (segment (start 128 45.83) (end 129.93 45.83) (width 0.25) (layer F.Cu) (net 18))
 (segment (start 130.39998 46.29998) (end 130.39998 59.00002) (width 0.25) (layer F.Cu) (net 18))
 (segment (start 129.93 45.83) (end 130.39998 46.29998) (width 0.25) (layer F.Cu) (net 18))
 (segment (start 130.39998 59.00002) (end 129.7 59.7) (width 0.25) (layer F.Cu) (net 18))
 (segment (start 118.805001 65.674999) (end 117.63 66.85) (width 0.25) (layer F.Cu) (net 18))
 (segment (start 118.805001 63.844999) (end 118.805001 65.674999) (width 0.25) (layer F.Cu) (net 18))
 (segment (start 122.95 59.7) (end 118.805001 63.844999) (width 0.25) (layer F.Cu) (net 18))
 (segment (start 129.7 59.7) (end 122.95 59.7) (width 0.25) (layer F.Cu) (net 18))
 (segment (start 128 48.37) (end 129.67 48.37) (width 0.25) (layer F.Cu) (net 19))
 (segment (start 129.67 48.37) (end 129.7 48.4) (width 0.25) (layer F.Cu) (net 19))
 (segment (start 129.7 48.4) (end 129.7 58.5) (width 0.25) (layer F.Cu) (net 19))
 (segment (start 129.7 58.5) (end 129.15 59.05) (width 0.25) (layer F.Cu) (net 19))
 (segment (start 116.265001 65.674999) (end 115.09 66.85) (width 0.25) (layer F.Cu) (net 19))
 (segment (start 116.265001 63.935997) (end 116.265001 65.674999) (width 0.25) (layer F.Cu) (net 19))
 (segment (start 121.150998 59.05) (end 116.265001 63.935997) (width 0.25) (layer F.Cu) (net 19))
 (segment (start 129.15 59.05) (end 121.150998 59.05) (width 0.25) (layer F.Cu) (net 19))
 (segment (start 149.474999 65.674999) (end 150.65 66.85) (width 0.25) (layer F.Cu) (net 10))
 (segment (start 149.474999 62.374999) (end 149.474999 65.674999) (width 0.25) (layer F.Cu) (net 10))
 (segment (start 148.3 61.2) (end 149.474999 62.374999) (width 0.25) (layer F.Cu) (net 10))
 (segment (start 144.7 61.2) (end 148.3 61.2) (width 0.25) (layer F.Cu) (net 10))
 (segment (start 143.25 50.9) (end 143.25 59.75) (width 0.25) (layer F.Cu) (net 10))
 (segment (start 143.25 59.75) (end 144.7 61.2) (width 0.25) (layer F.Cu) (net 10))
 (segment (start 128 40.75) (end 130.85 40.75) (width 0.25) (layer F.Cu) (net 16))
 (segment (start 130.85 40.75) (end 131.3 41.2) (width 0.25) (layer F.Cu) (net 16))
 (segment (start 131.3 41.2) (end 131.3 60.85) (width 0.25) (layer F.Cu) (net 16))
 (segment (start 131.3 60.85) (end 130.7 61.45) (width 0.25) (layer F.Cu) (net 16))
 (segment (start 130.7 61.45) (end 127.4 61.45) (width 0.25) (layer F.Cu) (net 16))
 (segment (start 127.4 61.45) (end 126.6 62.25) (width 0.25) (layer F.Cu) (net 16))
 (segment (start 126.6 65.5) (end 125.25 66.85) (width 0.25) (layer F.Cu) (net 16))
 (segment (start 126.6 62.25) (end 126.6 65.5) (width 0.25) (layer F.Cu) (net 16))
 (segment (start 128 43.29) (end 129.99 43.29) (width 0.25) (layer F.Cu) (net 17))
 (segment (start 129.99 43.29) (end 130.84999 44.14999) (width 0.25) (layer F.Cu) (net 17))
 (segment (start 130.84999 44.14999) (end 130.84999 59.90001) (width 0.25) (layer F.Cu) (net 17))
 (segment (start 130.84999 59.90001) (end 130.2 60.55) (width 0.25) (layer F.Cu) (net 17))
 (segment (start 130.2 60.55) (end 123.55 60.55) (width 0.25) (layer F.Cu) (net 17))
 (segment (start 121.534999 62.565001) (end 121.534999 65.565001) (width 0.25) (layer F.Cu) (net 17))
 (segment (start 123.55 60.55) (end 121.534999 62.565001) (width 0.25) (layer F.Cu) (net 17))
 (segment (start 120.25 66.85) (end 120.17 66.85) (width 0.25) (layer F.Cu) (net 17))
 (segment (start 121.534999 65.565001) (end 120.25 66.85) (width 0.25) (layer F.Cu) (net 17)))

